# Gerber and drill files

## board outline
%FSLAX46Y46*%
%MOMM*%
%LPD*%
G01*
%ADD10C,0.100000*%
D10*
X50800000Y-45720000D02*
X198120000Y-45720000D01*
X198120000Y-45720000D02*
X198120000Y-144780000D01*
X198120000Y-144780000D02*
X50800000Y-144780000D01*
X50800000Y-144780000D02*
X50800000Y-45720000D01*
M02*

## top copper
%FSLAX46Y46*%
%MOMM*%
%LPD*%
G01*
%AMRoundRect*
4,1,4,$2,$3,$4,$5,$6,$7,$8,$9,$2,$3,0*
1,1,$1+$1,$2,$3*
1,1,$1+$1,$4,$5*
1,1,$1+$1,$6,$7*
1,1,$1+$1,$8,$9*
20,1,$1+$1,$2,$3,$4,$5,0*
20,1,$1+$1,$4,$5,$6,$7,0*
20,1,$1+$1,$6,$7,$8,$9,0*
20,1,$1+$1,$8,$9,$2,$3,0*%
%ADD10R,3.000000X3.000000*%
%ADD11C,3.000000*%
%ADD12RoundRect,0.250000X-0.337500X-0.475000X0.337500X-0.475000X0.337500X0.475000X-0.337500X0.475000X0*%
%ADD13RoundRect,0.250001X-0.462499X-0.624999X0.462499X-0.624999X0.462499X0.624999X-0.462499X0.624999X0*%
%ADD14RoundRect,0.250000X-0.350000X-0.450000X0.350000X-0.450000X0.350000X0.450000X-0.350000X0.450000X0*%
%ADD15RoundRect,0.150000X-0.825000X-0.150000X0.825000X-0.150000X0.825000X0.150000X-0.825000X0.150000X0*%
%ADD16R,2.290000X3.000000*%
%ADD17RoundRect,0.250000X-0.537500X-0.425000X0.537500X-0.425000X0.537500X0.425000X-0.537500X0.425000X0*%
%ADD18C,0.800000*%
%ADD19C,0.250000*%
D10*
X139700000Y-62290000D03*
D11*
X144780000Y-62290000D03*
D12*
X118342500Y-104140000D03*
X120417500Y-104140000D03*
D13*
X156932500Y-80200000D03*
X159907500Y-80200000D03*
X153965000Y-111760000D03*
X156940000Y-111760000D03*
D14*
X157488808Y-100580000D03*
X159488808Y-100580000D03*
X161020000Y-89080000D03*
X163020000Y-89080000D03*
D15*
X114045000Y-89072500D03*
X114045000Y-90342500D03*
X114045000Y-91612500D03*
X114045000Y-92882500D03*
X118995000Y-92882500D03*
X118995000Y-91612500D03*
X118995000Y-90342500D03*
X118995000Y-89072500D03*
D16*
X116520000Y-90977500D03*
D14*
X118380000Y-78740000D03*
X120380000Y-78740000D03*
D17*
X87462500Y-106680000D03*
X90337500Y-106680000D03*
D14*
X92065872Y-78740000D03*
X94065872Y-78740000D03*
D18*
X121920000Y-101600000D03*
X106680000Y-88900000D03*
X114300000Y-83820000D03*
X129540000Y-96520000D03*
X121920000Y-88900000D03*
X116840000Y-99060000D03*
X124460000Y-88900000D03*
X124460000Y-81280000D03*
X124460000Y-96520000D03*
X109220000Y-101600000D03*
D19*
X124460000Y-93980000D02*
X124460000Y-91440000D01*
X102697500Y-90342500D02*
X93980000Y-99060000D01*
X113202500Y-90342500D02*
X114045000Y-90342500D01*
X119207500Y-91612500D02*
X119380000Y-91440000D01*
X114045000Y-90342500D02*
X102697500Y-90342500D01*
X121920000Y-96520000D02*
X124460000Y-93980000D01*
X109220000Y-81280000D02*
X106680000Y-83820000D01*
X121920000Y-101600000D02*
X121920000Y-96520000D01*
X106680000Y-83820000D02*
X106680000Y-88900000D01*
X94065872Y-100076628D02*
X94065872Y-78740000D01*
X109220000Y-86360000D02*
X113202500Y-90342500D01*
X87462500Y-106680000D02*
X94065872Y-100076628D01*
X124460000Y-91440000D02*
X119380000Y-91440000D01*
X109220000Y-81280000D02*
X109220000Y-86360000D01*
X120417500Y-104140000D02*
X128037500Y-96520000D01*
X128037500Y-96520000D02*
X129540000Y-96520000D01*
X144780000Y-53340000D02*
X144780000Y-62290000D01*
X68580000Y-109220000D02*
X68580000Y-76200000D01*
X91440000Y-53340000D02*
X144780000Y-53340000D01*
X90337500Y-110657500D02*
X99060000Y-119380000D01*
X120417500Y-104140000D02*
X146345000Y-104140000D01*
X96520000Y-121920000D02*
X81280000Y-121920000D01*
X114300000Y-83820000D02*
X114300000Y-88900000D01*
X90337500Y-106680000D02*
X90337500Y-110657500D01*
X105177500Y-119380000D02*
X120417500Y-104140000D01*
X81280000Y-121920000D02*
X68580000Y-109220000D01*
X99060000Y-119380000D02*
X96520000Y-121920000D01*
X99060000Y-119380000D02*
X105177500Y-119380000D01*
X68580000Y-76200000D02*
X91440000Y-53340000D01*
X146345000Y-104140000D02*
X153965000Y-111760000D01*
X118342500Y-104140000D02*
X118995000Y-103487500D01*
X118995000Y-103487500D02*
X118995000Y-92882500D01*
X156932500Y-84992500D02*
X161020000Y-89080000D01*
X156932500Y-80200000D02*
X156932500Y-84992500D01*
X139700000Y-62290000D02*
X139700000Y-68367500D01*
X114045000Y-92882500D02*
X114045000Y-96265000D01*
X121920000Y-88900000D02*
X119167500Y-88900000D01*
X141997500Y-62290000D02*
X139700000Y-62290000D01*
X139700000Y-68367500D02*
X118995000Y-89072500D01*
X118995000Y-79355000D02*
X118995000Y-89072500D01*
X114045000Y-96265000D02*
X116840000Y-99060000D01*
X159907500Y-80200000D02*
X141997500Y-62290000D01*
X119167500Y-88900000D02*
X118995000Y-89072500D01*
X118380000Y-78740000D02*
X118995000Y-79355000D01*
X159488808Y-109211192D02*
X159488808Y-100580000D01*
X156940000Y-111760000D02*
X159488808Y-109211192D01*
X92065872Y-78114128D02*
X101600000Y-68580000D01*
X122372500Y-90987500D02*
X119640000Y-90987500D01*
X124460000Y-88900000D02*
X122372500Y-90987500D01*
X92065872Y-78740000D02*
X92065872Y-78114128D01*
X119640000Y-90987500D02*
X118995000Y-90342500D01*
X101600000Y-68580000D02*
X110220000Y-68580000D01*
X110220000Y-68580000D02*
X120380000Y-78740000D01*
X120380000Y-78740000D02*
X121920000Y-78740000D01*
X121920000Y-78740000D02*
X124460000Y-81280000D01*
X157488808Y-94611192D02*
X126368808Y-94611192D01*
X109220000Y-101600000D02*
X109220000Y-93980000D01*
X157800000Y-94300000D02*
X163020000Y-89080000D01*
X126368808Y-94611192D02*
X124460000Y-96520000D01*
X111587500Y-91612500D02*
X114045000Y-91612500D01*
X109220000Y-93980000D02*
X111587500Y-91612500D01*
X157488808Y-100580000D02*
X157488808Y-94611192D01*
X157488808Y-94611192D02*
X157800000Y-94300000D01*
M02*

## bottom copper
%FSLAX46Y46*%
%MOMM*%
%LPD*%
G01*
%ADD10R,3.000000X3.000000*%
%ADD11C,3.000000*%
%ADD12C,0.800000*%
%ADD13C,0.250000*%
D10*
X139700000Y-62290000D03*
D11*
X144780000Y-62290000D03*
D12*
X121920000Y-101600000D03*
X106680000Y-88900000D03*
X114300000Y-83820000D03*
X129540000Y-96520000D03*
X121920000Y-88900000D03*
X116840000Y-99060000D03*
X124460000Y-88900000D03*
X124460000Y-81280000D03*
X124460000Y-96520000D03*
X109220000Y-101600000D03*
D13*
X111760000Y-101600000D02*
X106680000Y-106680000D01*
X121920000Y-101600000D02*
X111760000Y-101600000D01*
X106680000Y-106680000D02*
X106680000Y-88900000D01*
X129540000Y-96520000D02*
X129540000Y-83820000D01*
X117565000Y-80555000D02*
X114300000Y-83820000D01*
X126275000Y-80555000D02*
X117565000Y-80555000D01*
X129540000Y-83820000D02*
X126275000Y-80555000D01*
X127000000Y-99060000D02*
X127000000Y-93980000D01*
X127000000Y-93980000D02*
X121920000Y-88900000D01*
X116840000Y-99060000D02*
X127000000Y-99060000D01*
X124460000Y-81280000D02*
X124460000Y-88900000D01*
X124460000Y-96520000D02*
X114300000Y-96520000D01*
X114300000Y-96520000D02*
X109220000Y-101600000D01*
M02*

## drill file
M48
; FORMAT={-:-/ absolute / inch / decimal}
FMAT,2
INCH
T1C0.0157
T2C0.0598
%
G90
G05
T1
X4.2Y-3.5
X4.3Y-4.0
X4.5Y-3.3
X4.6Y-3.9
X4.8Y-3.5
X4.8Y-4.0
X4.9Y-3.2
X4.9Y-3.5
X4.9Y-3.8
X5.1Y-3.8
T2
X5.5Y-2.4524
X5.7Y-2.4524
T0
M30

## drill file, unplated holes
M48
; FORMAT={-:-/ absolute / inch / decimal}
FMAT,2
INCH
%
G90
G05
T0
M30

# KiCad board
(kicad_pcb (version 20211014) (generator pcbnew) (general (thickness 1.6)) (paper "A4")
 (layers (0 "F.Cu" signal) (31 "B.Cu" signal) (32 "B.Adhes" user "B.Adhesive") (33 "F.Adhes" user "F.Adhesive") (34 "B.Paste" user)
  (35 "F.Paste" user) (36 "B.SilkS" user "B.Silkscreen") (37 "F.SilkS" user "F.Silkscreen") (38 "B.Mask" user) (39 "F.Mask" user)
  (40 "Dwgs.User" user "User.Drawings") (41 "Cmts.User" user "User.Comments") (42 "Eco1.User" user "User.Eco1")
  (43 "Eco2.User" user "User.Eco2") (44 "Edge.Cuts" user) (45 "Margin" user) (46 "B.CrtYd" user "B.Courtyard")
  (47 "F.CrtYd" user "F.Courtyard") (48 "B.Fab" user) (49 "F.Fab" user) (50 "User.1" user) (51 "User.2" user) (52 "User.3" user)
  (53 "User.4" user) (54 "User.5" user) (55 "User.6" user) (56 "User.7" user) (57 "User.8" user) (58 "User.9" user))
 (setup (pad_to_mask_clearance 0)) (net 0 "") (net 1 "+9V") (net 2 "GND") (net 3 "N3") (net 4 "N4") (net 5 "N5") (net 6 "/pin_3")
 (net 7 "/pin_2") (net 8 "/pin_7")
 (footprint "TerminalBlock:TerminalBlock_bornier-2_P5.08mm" (layer "F.Cu") (at 139.7 62.29)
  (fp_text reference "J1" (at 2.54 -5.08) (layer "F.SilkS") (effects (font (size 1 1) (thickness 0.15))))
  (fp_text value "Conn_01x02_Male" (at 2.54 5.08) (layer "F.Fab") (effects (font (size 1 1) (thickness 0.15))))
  (pad "1" thru_hole rect (at 0 0) (size 3 3) (drill 1.52) (layers *.Cu *.Mask) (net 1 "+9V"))
  (pad "2" thru_hole circle (at 5.08 0) (size 3 3) (drill 1.52) (layers *.Cu *.Mask) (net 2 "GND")))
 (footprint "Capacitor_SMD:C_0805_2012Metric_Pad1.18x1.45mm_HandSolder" (layer "F.Cu") (at 119.38 104.14)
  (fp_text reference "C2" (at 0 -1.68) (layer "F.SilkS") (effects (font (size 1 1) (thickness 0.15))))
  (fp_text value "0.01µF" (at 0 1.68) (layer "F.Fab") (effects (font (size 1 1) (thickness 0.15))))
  (pad "1" smd roundrect (at -1.0375 0) (size 1.175 1.45) (layers "F.Cu" "F.Paste" "F.Mask") (roundrect_rratio 0.2127659574) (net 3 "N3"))
  (pad "2" smd roundrect (at 1.0375 0) (size 1.175 1.45) (layers "F.Cu" "F.Paste" "F.Mask") (roundrect_rratio 0.2127659574) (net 2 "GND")))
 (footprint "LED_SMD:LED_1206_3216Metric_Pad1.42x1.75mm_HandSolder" (layer "F.Cu") (at 158.42 80.2)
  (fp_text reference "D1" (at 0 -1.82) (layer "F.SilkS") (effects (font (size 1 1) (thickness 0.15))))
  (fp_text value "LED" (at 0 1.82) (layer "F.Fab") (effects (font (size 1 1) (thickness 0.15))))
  (pad "1" smd roundrect (at -1.4875 0) (size 1.425 1.75) (layers "F.Cu" "F.Paste" "F.Mask") (roundrect_rratio 0.1754392982) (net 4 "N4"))
  (pad "2" smd roundrect (at 1.4875 0) (size 1.425 1.75) (layers "F.Cu" "F.Paste" "F.Mask") (roundrect_rratio 0.1754392982) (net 1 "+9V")))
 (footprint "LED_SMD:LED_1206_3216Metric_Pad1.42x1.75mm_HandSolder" (layer "F.Cu") (at 155.4525 111.76)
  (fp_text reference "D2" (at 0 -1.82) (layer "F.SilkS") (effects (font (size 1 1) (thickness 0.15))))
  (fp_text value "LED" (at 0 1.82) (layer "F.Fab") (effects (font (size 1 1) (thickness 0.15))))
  (pad "1" smd roundrect (at -1.4875 0) (size 1.425 1.75) (layers "F.Cu" "F.Paste" "F.Mask") (roundrect_rratio 0.1754392982) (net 2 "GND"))
  (pad "2" smd roundrect (at 1.4875 0) (size 1.425 1.75) (layers "F.Cu" "F.Paste" "F.Mask") (roundrect_rratio 0.1754392982) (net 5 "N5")))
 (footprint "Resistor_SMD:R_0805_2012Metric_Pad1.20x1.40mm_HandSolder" (layer "F.Cu") (at 158.488808 100.58)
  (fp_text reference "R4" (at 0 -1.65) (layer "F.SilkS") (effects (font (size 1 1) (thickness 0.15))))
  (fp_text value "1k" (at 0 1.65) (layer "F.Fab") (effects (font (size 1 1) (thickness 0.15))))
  (pad "1" smd roundrect (at -1 0) (size 1.2 1.4) (layers "F.Cu" "F.Paste" "F.Mask") (roundrect_rratio 0.2083333333) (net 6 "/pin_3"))
  (pad "2" smd roundrect (at 1 0) (size 1.2 1.4) (layers "F.Cu" "F.Paste" "F.Mask") (roundrect_rratio 0.2083333333) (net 5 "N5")))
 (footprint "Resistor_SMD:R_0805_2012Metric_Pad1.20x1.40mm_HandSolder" (layer "F.Cu") (at 162.02 89.08)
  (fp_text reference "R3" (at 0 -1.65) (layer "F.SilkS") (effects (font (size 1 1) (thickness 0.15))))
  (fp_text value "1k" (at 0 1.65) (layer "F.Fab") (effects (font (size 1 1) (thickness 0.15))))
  (pad "1" smd roundrect (at -1 0) (size 1.2 1.4) (layers "F.Cu" "F.Paste" "F.Mask") (roundrect_rratio 0.2083333333) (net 4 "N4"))
  (pad "2" smd roundrect (at 1 0) (size 1.2 1.4) (layers "F.Cu" "F.Paste" "F.Mask") (roundrect_rratio 0.2083333333) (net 6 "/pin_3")))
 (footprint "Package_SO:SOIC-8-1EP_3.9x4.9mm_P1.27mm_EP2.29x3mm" (layer "F.Cu") (at 116.52 90.9775)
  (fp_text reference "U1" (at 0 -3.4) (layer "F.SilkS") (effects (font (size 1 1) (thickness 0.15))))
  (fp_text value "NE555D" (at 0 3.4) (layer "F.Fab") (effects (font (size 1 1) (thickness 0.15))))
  (pad "" smd roundrect (at 0.57 -0.75) (size 0.92 1.21) (layers "F.Paste") (roundrect_rratio 0.25))
  (pad "" smd roundrect (at 0.57 0.75) (size 0.92 1.21) (layers "F.Paste") (roundrect_rratio 0.25))
  (pad "" smd roundrect (at -0.57 0.75) (size 0.92 1.21) (layers "F.Paste") (roundrect_rratio 0.25))
  (pad "" smd roundrect (at -0.57 -0.75) (size 0.92 1.21) (layers "F.Paste") (roundrect_rratio 0.25))
  (pad "1" smd roundrect (at -2.475 -1.905) (size 1.95 0.6) (layers "F.Cu" "F.Paste" "F.Mask") (roundrect_rratio 0.25) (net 2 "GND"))
  (pad "2" smd roundrect (at -2.475 -0.635) (size 1.95 0.6) (layers "F.Cu" "F.Paste" "F.Mask") (roundrect_rratio 0.25) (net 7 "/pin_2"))
  (pad "3" smd roundrect (at -2.475 0.635) (size 1.95 0.6) (layers "F.Cu" "F.Paste" "F.Mask") (roundrect_rratio 0.25) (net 6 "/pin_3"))
  (pad "4" smd roundrect (at -2.475 1.905) (size 1.95 0.6) (layers "F.Cu" "F.Paste" "F.Mask") (roundrect_rratio 0.25) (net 1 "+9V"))
  (pad "5" smd roundrect (at 2.475 1.905) (size 1.95 0.6) (layers "F.Cu" "F.Paste" "F.Mask") (roundrect_rratio 0.25) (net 3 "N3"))
  (pad "6" smd roundrect (at 2.475 0.635) (size 1.95 0.6) (layers "F.Cu" "F.Paste" "F.Mask") (roundrect_rratio 0.25) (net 7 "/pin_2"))
  (pad "7" smd roundrect (at 2.475 -0.635) (size 1.95 0.6) (layers "F.Cu" "F.Paste" "F.Mask") (roundrect_rratio 0.25) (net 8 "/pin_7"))
  (pad "8" smd roundrect (at 2.475 -1.905) (size 1.95 0.6) (layers "F.Cu" "F.Paste" "F.Mask") (roundrect_rratio 0.25) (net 1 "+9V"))
  (pad "9" smd rect (at 0 0) (size 2.29 3) (layers "F.Cu" "F.Mask")))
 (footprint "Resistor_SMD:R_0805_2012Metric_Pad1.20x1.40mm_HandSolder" (layer "F.Cu") (at 119.38 78.74)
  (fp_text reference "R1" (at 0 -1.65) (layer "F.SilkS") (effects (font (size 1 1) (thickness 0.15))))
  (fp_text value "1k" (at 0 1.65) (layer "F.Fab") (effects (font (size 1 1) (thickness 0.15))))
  (pad "1" smd roundrect (at -1 0) (size 1.2 1.4) (layers "F.Cu" "F.Paste" "F.Mask") (roundrect_rratio 0.2083333333) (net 1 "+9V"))
  (pad "2" smd roundrect (at 1 0) (size 1.2 1.4) (layers "F.Cu" "F.Paste" "F.Mask") (roundrect_rratio 0.2083333333) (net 8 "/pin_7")))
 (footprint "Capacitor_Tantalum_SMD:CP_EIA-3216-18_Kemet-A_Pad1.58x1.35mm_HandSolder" (layer "F.Cu") (at 88.9 106.68)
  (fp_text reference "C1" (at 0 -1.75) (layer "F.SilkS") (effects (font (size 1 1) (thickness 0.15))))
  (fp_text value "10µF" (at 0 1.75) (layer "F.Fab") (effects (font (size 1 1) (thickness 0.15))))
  (pad "1" smd roundrect (at -1.4375 0) (size 1.575 1.35) (layers "F.Cu" "F.Paste" "F.Mask") (roundrect_rratio 0.1851851852)
   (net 7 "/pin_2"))
  (pad "2" smd roundrect (at 1.4375 0) (size 1.575 1.35) (layers "F.Cu" "F.Paste" "F.Mask") (roundrect_rratio 0.1851851852) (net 2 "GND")))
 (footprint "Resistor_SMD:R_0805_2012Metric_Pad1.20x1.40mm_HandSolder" (layer "F.Cu") (at 93.065872 78.74)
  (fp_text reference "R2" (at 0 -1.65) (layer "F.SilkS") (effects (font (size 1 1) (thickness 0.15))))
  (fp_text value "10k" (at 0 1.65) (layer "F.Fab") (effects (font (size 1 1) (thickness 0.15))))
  (pad "1" smd roundrect (at -1 0) (size 1.2 1.4) (layers "F.Cu" "F.Paste" "F.Mask") (roundrect_rratio 0.2083333333) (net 8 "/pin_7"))
  (pad "2" smd roundrect (at 1 0) (size 1.2 1.4) (layers "F.Cu" "F.Paste" "F.Mask") (roundrect_rratio 0.2083333333) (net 7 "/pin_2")))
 (gr_rect (start 50.8 45.72) (end 198.12 144.78) (layer "Edge.Cuts") (width 0.1) (fill none))
 (segment (start 124.46 93.98) (end 124.46 91.44) (width 0.25) (layer "F.Cu") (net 7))
 (segment (start 102.6975 90.3425) (end 93.98 99.06) (width 0.25) (layer "F.Cu") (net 7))
 (segment (start 113.2025 90.3425) (end 114.045 90.3425) (width 0.25) (layer "F.Cu") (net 7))
 (segment (start 119.2075 91.6125) (end 119.38 91.44) (width 0.25) (layer "F.Cu") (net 7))
 (segment (start 114.045 90.3425) (end 102.6975 90.3425) (width 0.25) (layer "F.Cu") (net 7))
 (segment (start 121.92 96.52) (end 124.46 93.98) (width 0.25) (layer "F.Cu") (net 7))
 (segment (start 109.22 81.28) (end 106.68 83.82) (width 0.25) (layer "F.Cu") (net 7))
 (segment (start 121.92 101.6) (end 121.92 96.52) (width 0.25) (layer "F.Cu") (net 7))
 (segment (start 106.68 83.82) (end 106.68 88.9) (width 0.25) (layer "F.Cu") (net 7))
 (segment (start 94.065872 100.076628) (end 94.065872 78.74) (width 0.25) (layer "F.Cu") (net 7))
 (segment (start 109.22 86.36) (end 113.2025 90.3425) (width 0.25) (layer "F.Cu") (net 7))
 (segment (start 87.4625 106.68) (end 94.065872 100.076628) (width 0.25) (layer "F.Cu") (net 7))
 (segment (start 124.46 91.44) (end 119.38 91.44) (width 0.25) (layer "F.Cu") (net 7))
 (segment (start 109.22 81.28) (end 109.22 86.36) (width 0.25) (layer "F.Cu") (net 7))
 (via (at 121.92 101.6) (size 0.8) (drill 0.4) (layers "F.Cu" "B.Cu") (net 7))
 (via (at 106.68 88.9) (size 0.8) (drill 0.4) (layers "F.Cu" "B.Cu") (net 7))
 (segment (start 111.76 101.6) (end 106.68 106.68) (width 0.25) (layer "B.Cu") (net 7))
 (segment (start 121.92 101.6) (end 111.76 101.6) (width 0.25) (layer "B.Cu") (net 7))
 (segment (start 106.68 106.68) (end 106.68 88.9) (width 0.25) (layer "B.Cu") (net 7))
 (segment (start 120.4175 104.14) (end 128.0375 96.52) (width 0.25) (layer "F.Cu") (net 2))
 (segment (start 128.0375 96.52) (end 129.54 96.52) (width 0.25) (layer "F.Cu") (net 2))
 (segment (start 144.78 53.34) (end 144.78 62.29) (width 0.25) (layer "F.Cu") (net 2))
 (segment (start 68.58 109.22) (end 68.58 76.2) (width 0.25) (layer "F.Cu") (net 2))
 (segment (start 91.44 53.34) (end 144.78 53.34) (width 0.25) (layer "F.Cu") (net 2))
 (segment (start 90.3375 110.6575) (end 99.06 119.38) (width 0.25) (layer "F.Cu") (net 2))
 (segment (start 120.4175 104.14) (end 146.345 104.14) (width 0.25) (layer "F.Cu") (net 2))
 (segment (start 96.52 121.92) (end 81.28 121.92) (width 0.25) (layer "F.Cu") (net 2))
 (segment (start 114.3 83.82) (end 114.3 88.9) (width 0.25) (layer "F.Cu") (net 2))
 (segment (start 90.3375 106.68) (end 90.3375 110.6575) (width 0.25) (layer "F.Cu") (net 2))
 (segment (start 105.1775 119.38) (end 120.4175 104.14) (width 0.25) (layer "F.Cu") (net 2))
 (segment (start 81.28 121.92) (end 68.58 109.22) (width 0.25) (layer "F.Cu") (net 2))
 (segment (start 99.06 119.38) (end 96.52 121.92) (width 0.25) (layer "F.Cu") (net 2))
 (segment (start 99.06 119.38) (end 105.1775 119.38) (width 0.25) (layer "F.Cu") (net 2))
 (segment (start 68.58 76.2) (end 91.44 53.34) (width 0.25) (layer "F.Cu") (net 2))
 (segment (start 146.345 104.14) (end 153.965 111.76) (width 0.25) (layer "F.Cu") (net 2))
 (via (at 114.3 83.82) (size 0.8) (drill 0.4) (layers "F.Cu" "B.Cu") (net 2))
 (via (at 129.54 96.52) (size 0.8) (drill 0.4) (layers "F.Cu" "B.Cu") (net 2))
 (segment (start 129.54 96.52) (end 129.54 83.82) (width 0.25) (layer "B.Cu") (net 2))
 (segment (start 117.565 80.555) (end 114.3 83.82) (width 0.25) (layer "B.Cu") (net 2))
 (segment (start 126.275 80.555) (end 117.565 80.555) (width 0.25) (layer "B.Cu") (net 2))
 (segment (start 129.54 83.82) (end 126.275 80.555) (width 0.25) (layer "B.Cu") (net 2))
 (segment (start 118.3425 104.14) (end 118.995 103.4875) (width 0.25) (layer "F.Cu") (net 3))
 (segment (start 118.995 103.4875) (end 118.995 92.8825) (width 0.25) (layer "F.Cu") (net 3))
 (segment (start 156.9325 84.9925) (end 161.02 89.08) (width 0.25) (layer "F.Cu") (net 4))
 (segment (start 156.9325 80.2) (end 156.9325 84.9925) (width 0.25) (layer "F.Cu") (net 4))
 (segment (start 139.7 62.29) (end 139.7 68.3675) (width 0.25) (layer "F.Cu") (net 1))
 (segment (start 114.045 92.8825) (end 114.045 96.265) (width 0.25) (layer "F.Cu") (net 1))
 (segment (start 121.92 88.9) (end 119.1675 88.9) (width 0.25) (layer "F.Cu") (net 1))
 (segment (start 141.9975 62.29) (end 139.7 62.29) (width 0.25) (layer "F.Cu") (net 1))
 (segment (start 139.7 68.3675) (end 118.995 89.0725) (width 0.25) (layer "F.Cu") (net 1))
 (segment (start 118.995 79.355) (end 118.995 89.0725) (width 0.25) (layer "F.Cu") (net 1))
 (segment (start 114.045 96.265) (end 116.84 99.06) (width 0.25) (layer "F.Cu") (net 1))
 (segment (start 159.9075 80.2) (end 141.9975 62.29) (width 0.25) (layer "F.Cu") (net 1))
 (segment (start 119.1675 88.9) (end 118.995 89.0725) (width 0.25) (layer "F.Cu") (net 1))
 (segment (start 118.38 78.74) (end 118.995 79.355) (width 0.25) (layer "F.Cu") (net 1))
 (via (at 121.92 88.9) (size 0.8) (drill 0.4) (layers "F.Cu" "B.Cu") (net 1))
 (via (at 116.84 99.06) (size 0.8) (drill 0.4) (layers "F.Cu" "B.Cu") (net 1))
 (segment (start 127 99.06) (end 127 93.98) (width 0.25) (layer "B.Cu") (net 1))
 (segment (start 127 93.98) (end 121.92 88.9) (width 0.25) (layer "B.Cu") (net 1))
 (segment (start 116.84 99.06) (end 127 99.06) (width 0.25) (layer "B.Cu") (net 1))
 (segment (start 159.488808 109.211192) (end 159.488808 100.58) (width 0.25) (layer "F.Cu") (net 5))
 (segment (start 156.94 111.76) (end 159.488808 109.211192) (width 0.25) (layer "F.Cu") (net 5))
 (segment (start 92.065872 78.114128) (end 101.6 68.58) (width 0.25) (layer "F.Cu") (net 8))
 (segment (start 122.3725 90.9875) (end 119.64 90.9875) (width 0.25) (layer "F.Cu") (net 8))
 (segment (start 124.46 88.9) (end 122.3725 90.9875) (width 0.25) (layer "F.Cu") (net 8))
 (segment (start 92.065872 78.74) (end 92.065872 78.114128) (width 0.25) (layer "F.Cu") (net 8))
 (segment (start 119.64 90.9875) (end 118.995 90.3425) (width 0.25) (layer "F.Cu") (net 8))
 (segment (start 101.6 68.58) (end 110.22 68.58) (width 0.25) (layer "F.Cu") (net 8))
 (segment (start 110.22 68.58) (end 120.38 78.74) (width 0.25) (layer "F.Cu") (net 8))
 (segment (start 120.38 78.74) (end 121.92 78.74) (width 0.25) (layer "F.Cu") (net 8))
 (segment (start 121.92 78.74) (end 124.46 81.28) (width 0.25) (layer "F.Cu") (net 8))
 (via (at 124.46 88.9) (size 0.8) (drill 0.4) (layers "F.Cu" "B.Cu") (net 8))
 (via (at 124.46 81.28) (size 0.8) (drill 0.4) (layers "F.Cu" "B.Cu") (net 8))
 (segment (start 124.46 81.28) (end 124.46 88.9) (width 0.25) (layer "B.Cu") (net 8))
 (segment (start 157.488808 94.611192) (end 126.368808 94.611192) (width 0.25) (layer "F.Cu") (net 6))
 (segment (start 109.22 101.6) (end 109.22 93.98) (width 0.25) (layer "F.Cu") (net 6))
 (segment (start 157.8 94.3) (end 163.02 89.08) (width 0.25) (layer "F.Cu") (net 6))
 (segment (start 126.368808 94.611192) (end 124.46 96.52) (width 0.25) (layer "F.Cu") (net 6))
 (segment (start 111.5875 91.6125) (end 114.045 91.6125) (width 0.25) (layer "F.Cu") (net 6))
 (segment (start 109.22 93.98) (end 111.5875 91.6125) (width 0.25) (layer "F.Cu") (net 6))
 (segment (start 157.488808 100.58) (end 157.488808 94.611192) (width 0.25) (layer "F.Cu") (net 6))
 (segment (start 157.488808 94.611192) (end 157.8 94.3) (width 0.25) (layer "F.Cu") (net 6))
 (via (at 124.46 96.52) (size 0.8) (drill 0.4) (layers "F.Cu" "B.Cu") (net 6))
 (via (at 109.22 101.6) (size 0.8) (drill 0.4) (layers "F.Cu" "B.Cu") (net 6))
 (segment (start 124.46 96.52) (end 114.3 96.52) (width 0.25) (layer "B.Cu") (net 6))
 (segment (start 114.3 96.52) (end 109.22 101.6) (width 0.25) (layer "B.Cu") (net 6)))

